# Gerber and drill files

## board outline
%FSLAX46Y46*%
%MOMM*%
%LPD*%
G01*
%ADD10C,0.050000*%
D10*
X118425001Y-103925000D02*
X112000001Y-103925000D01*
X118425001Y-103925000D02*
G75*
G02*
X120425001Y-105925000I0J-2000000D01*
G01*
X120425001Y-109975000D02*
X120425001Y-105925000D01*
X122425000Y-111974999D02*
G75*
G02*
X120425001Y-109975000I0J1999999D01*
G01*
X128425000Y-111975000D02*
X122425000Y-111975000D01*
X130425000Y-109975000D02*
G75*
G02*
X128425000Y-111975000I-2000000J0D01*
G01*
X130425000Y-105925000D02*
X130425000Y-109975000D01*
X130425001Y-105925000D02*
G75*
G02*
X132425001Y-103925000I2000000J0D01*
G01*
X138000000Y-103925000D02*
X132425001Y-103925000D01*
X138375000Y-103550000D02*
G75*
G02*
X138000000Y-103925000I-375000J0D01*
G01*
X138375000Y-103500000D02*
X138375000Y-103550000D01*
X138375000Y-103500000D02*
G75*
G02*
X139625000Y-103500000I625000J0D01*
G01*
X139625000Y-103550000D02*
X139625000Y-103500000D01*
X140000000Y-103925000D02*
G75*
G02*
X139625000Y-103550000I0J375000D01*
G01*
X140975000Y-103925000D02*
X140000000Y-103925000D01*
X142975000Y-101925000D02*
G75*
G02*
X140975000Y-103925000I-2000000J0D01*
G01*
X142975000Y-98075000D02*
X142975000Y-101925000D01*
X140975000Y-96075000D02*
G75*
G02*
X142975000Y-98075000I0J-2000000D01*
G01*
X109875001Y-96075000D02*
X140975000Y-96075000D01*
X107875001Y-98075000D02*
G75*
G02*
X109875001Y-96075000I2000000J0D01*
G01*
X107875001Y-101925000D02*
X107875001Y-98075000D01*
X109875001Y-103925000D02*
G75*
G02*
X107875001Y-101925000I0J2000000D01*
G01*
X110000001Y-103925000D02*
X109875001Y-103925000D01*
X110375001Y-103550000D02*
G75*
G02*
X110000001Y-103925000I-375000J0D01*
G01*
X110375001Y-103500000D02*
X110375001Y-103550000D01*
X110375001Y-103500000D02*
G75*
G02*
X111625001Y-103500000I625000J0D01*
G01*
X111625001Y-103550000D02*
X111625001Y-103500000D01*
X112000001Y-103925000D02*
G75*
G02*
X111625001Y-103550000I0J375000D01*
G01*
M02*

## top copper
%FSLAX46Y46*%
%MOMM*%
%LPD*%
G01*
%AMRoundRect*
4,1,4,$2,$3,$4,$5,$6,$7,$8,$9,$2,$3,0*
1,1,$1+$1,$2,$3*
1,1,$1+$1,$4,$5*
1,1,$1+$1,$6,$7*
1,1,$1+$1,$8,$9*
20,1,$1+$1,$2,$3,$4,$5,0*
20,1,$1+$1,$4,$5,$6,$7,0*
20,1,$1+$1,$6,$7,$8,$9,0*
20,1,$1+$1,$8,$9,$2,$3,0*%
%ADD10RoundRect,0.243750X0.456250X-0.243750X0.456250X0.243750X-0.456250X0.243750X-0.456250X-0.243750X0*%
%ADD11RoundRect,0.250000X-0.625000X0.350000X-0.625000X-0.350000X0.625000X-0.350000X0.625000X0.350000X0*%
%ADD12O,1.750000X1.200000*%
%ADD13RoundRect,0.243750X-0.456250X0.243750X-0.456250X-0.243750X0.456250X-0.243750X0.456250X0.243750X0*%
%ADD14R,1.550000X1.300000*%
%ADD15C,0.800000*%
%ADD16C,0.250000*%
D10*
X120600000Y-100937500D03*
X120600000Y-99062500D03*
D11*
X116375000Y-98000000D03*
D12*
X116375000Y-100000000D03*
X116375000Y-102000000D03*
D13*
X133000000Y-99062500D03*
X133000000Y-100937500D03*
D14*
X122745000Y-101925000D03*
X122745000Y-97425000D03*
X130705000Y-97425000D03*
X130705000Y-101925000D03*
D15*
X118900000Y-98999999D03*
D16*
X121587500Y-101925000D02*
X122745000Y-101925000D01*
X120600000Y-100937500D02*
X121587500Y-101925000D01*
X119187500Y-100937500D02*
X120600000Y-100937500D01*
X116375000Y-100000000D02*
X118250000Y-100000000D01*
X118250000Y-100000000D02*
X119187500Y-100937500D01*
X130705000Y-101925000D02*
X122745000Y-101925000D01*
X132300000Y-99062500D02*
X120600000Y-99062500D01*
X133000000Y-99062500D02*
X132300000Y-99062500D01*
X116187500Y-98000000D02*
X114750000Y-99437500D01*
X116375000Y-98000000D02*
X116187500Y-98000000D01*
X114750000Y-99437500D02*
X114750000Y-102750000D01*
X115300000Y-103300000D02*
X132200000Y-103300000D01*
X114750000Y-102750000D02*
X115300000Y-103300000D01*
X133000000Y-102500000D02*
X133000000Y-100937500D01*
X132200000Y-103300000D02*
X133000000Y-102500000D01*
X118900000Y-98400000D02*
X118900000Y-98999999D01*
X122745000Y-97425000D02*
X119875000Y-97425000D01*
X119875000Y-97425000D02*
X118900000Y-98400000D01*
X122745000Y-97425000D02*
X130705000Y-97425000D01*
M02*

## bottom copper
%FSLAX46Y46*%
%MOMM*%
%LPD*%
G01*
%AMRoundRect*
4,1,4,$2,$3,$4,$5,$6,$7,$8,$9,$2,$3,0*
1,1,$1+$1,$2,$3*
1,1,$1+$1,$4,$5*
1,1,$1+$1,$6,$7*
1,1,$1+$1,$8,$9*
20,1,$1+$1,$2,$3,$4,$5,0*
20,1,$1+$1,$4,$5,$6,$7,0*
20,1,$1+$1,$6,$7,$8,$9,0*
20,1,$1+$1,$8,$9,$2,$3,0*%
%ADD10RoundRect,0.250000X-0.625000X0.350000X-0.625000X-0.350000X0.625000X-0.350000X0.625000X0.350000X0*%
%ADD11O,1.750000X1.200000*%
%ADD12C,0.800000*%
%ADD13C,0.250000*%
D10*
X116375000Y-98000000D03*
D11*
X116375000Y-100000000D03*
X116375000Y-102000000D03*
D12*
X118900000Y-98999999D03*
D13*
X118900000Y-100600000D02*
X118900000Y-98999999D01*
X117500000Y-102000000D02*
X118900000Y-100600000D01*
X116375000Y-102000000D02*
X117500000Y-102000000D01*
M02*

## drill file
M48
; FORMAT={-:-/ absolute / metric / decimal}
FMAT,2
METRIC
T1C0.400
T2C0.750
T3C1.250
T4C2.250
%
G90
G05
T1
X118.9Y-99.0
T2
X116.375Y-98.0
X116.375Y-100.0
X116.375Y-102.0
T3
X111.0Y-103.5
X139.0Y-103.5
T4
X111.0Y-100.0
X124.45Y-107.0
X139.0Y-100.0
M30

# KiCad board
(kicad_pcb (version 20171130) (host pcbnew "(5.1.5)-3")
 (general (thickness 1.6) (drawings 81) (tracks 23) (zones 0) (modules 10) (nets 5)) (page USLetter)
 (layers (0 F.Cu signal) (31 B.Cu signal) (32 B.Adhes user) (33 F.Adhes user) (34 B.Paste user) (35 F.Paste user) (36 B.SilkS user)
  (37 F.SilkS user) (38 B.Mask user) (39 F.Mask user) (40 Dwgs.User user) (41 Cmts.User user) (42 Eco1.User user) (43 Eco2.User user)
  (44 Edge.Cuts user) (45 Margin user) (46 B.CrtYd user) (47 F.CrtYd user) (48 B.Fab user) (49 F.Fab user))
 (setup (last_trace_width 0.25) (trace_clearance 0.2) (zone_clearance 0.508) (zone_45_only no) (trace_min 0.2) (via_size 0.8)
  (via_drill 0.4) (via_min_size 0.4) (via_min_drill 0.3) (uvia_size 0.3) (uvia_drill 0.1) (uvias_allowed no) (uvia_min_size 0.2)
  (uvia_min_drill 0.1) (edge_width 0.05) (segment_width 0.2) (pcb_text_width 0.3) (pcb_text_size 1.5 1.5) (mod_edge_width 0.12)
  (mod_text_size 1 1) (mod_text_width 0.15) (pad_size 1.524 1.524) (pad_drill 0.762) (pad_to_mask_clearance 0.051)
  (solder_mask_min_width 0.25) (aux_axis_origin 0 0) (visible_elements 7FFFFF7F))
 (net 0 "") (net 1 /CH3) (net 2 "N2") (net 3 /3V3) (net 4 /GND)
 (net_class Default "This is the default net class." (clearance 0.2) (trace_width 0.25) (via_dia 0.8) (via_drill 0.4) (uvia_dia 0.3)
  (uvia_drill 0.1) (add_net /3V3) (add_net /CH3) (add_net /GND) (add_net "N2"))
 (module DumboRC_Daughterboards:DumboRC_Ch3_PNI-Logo (layer B.Cu) (at 128.5 100.25 180)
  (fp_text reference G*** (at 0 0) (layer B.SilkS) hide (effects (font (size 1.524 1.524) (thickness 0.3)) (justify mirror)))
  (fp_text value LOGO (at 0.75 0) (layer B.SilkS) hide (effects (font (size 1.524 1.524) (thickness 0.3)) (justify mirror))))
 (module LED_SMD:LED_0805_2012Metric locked (layer F.Cu) (at 120.6 100 90)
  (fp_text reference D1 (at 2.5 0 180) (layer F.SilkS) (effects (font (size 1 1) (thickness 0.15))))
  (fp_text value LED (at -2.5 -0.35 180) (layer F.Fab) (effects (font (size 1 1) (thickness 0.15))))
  (pad 1 smd roundrect (at -0.9375 0 90) (size 0.975 1.4) (layers F.Cu F.Paste F.Mask) (roundrect_rratio 0.25) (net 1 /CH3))
  (pad 2 smd roundrect (at 0.9375 0 90) (size 0.975 1.4) (layers F.Cu F.Paste F.Mask) (roundrect_rratio 0.25) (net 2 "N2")))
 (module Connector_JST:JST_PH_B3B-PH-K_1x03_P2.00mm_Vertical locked (layer F.Cu) (at 116.375 98 270)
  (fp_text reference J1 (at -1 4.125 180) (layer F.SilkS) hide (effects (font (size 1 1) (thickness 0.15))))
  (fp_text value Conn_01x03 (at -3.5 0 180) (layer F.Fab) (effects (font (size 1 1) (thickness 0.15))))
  (pad 1 thru_hole roundrect (at 0 0 270) (size 1.2 1.75) (drill 0.75) (layers *.Cu *.Mask) (roundrect_rratio 0.208333) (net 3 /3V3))
  (pad 2 thru_hole oval (at 2 0 270) (size 1.2 1.75) (drill 0.75) (layers *.Cu *.Mask) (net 1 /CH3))
  (pad 3 thru_hole oval (at 4 0 270) (size 1.2 1.75) (drill 0.75) (layers *.Cu *.Mask) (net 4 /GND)))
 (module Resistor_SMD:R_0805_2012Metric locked (layer F.Cu) (at 133 100 270)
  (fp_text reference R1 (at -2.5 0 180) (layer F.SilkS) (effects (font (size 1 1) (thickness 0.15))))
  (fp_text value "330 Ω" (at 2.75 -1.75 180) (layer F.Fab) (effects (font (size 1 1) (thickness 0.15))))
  (pad 1 smd roundrect (at -0.9375 0 270) (size 0.975 1.4) (layers F.Cu F.Paste F.Mask) (roundrect_rratio 0.25) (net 2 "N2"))
  (pad 2 smd roundrect (at 0.9375 0 270) (size 0.975 1.4) (layers F.Cu F.Paste F.Mask) (roundrect_rratio 0.25) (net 3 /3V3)))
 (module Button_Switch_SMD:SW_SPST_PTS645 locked (layer F.Cu) (at 126.725 99.675)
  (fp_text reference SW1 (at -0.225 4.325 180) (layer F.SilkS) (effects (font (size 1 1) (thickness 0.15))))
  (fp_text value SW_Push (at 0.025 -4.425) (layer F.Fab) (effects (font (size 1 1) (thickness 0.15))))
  (pad 2 smd rect (at -3.98 2.25) (size 1.55 1.3) (layers F.Cu F.Paste F.Mask) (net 1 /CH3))
  (pad 1 smd rect (at -3.98 -2.25) (size 1.55 1.3) (layers F.Cu F.Paste F.Mask) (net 4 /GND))
  (pad 1 smd rect (at 3.98 -2.25) (size 1.55 1.3) (layers F.Cu F.Paste F.Mask) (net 4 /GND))
  (pad 2 smd rect (at 3.98 2.25) (size 1.55 1.3) (layers F.Cu F.Paste F.Mask) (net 1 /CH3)))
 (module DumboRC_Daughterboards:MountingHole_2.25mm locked (layer F.Cu) (at 111 100)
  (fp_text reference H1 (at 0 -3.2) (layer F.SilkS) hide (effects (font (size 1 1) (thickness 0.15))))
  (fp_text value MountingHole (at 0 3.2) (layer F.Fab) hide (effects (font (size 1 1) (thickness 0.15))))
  (pad "" np_thru_hole circle (at 0 0 90) (size 2.25 2.25) (drill 2.25) (layers *.Cu *.Mask)))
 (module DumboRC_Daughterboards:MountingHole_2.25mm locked (layer F.Cu) (at 139 100)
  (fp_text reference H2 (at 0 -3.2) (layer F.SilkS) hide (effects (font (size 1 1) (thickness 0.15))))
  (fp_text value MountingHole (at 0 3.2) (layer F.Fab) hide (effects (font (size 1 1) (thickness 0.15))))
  (pad "" np_thru_hole circle (at 0 0 90) (size 2.25 2.25) (drill 2.25) (layers *.Cu *.Mask)))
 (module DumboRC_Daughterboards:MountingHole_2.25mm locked (layer F.Cu) (at 124.45 107)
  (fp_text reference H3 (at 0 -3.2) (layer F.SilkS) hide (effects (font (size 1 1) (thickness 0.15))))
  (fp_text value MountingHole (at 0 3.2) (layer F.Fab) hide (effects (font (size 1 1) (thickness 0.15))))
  (pad "" np_thru_hole circle (at 0 0 90) (size 2.25 2.25) (drill 2.25) (layers *.Cu *.Mask)))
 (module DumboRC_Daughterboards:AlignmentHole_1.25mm (layer F.Cu) (at 111 103.5)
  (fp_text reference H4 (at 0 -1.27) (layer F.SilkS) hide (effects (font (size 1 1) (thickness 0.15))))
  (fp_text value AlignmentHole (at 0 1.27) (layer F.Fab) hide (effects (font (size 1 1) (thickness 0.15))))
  (pad "" np_thru_hole circle (at 0 0 90) (size 1.25 1.25) (drill 1.25) (layers *.Cu *.Mask)))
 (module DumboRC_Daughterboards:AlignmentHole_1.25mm (layer F.Cu) (at 139 103.5)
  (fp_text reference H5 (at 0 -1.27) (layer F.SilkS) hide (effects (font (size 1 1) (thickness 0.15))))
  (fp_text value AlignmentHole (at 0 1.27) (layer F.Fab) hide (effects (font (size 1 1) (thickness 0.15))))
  (pad "" np_thru_hole circle (at 0 0 90) (size 1.25 1.25) (drill 1.25) (layers *.Cu *.Mask)))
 (gr_line (start 118.425001 103.925) (end 112.000001 103.925) (layer Edge.Cuts) (width 0.05))
 (gr_arc (start 118.425001 105.925) (end 120.425001 105.925) (angle -90) (layer Edge.Cuts) (width 0.05))
 (gr_line (start 120.425001 109.975) (end 120.425001 105.925) (layer Edge.Cuts) (width 0.05))
 (gr_arc (start 122.425 109.975) (end 120.425001 109.975) (angle -90) (layer Edge.Cuts) (width 0.05))
 (gr_line (start 128.425 111.975) (end 122.425 111.975) (layer Edge.Cuts) (width 0.05))
 (gr_arc (start 128.425 109.975) (end 128.425 111.975) (angle -90) (layer Edge.Cuts) (width 0.05))
 (gr_line (start 130.425 105.925) (end 130.425 109.975) (layer Edge.Cuts) (width 0.05))
 (gr_arc (start 132.425001 105.925) (end 132.425001 103.925) (angle -90) (layer Edge.Cuts) (width 0.05))
 (gr_line (start 138 103.925) (end 132.425001 103.925) (layer Edge.Cuts) (width 0.05))
 (gr_arc (start 138 103.55) (end 138 103.925) (angle -90) (layer Edge.Cuts) (width 0.05))
 (gr_line (start 138.375 103.5) (end 138.375 103.55) (layer Edge.Cuts) (width 0.05))
 (gr_arc (start 139 103.5) (end 139.625 103.5) (angle -180) (layer Edge.Cuts) (width 0.05))
 (gr_line (start 139.625 103.55) (end 139.625 103.5) (layer Edge.Cuts) (width 0.05))
 (gr_arc (start 140 103.55) (end 139.625 103.55) (angle -90) (layer Edge.Cuts) (width 0.05))
 (gr_line (start 140.975 103.925) (end 140 103.925) (layer Edge.Cuts) (width 0.05))
 (gr_arc (start 140.975 101.925) (end 140.975 103.925) (angle -90) (layer Edge.Cuts) (width 0.05))
 (gr_line (start 142.975 98.075) (end 142.975 101.925) (layer Edge.Cuts) (width 0.05))
 (gr_arc (start 140.975 98.075) (end 142.975 98.075) (angle -90) (layer Edge.Cuts) (width 0.05))
 (gr_line (start 109.875001 96.075) (end 140.975 96.075) (layer Edge.Cuts) (width 0.05))
 (gr_arc (start 109.875001 98.075) (end 109.875001 96.075) (angle -90) (layer Edge.Cuts) (width 0.05))
 (gr_line (start 107.875001 101.925) (end 107.875001 98.075) (layer Edge.Cuts) (width 0.05))
 (gr_arc (start 109.875001 101.925) (end 107.875001 101.925) (angle -90) (layer Edge.Cuts) (width 0.05))
 (gr_line (start 110.000001 103.925) (end 109.875001 103.925) (layer Edge.Cuts) (width 0.05))
 (gr_arc (start 110.000001 103.55) (end 110.000001 103.925) (angle -90) (layer Edge.Cuts) (width 0.05))
 (gr_line (start 110.375001 103.5) (end 110.375001 103.55) (layer Edge.Cuts) (width 0.05))
 (gr_arc (start 111.000001 103.5) (end 111.625001 103.5) (angle -180) (layer Edge.Cuts) (width 0.05))
 (gr_line (start 111.625001 103.55) (end 111.625001 103.5) (layer Edge.Cuts) (width 0.05))
 (gr_arc (start 112.000001 103.55) (end 111.625001 103.55) (angle -90) (layer Edge.Cuts) (width 0.05))
 (segment (start 121.5875 101.925) (end 122.745 101.925) (width 0.25) (layer F.Cu) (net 1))
 (segment (start 120.6 100.9375) (end 121.5875 101.925) (width 0.25) (layer F.Cu) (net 1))
 (segment (start 119.1875 100.9375) (end 120.6 100.9375) (width 0.25) (layer F.Cu) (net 1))
 (segment (start 116.375 100) (end 118.25 100) (width 0.25) (layer F.Cu) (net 1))
 (segment (start 118.25 100) (end 119.1875 100.9375) (width 0.25) (layer F.Cu) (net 1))
 (segment (start 130.705 101.925) (end 122.745 101.925) (width 0.25) (layer F.Cu) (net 1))
 (segment (start 132.3 99.0625) (end 120.6 99.0625) (width 0.25) (layer F.Cu) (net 2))
 (segment (start 133 99.0625) (end 132.3 99.0625) (width 0.25) (layer F.Cu) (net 2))
 (segment (start 116.1875 98) (end 114.75 99.4375) (width 0.25) (layer F.Cu) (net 3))
 (segment (start 116.375 98) (end 116.1875 98) (width 0.25) (layer F.Cu) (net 3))
 (segment (start 114.75 99.4375) (end 114.75 102.75) (width 0.25) (layer F.Cu) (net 3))
 (segment (start 115.3 103.3) (end 132.2 103.3) (width 0.25) (layer F.Cu) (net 3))
 (segment (start 114.75 102.75) (end 115.3 103.3) (width 0.25) (layer F.Cu) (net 3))
 (segment (start 133 102.5) (end 133 100.9375) (width 0.25) (layer F.Cu) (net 3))
 (segment (start 132.2 103.3) (end 133 102.5) (width 0.25) (layer F.Cu) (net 3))
 (via (at 118.9 98.999999) (size 0.8) (drill 0.4) (layers F.Cu B.Cu) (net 4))
 (segment (start 118.9 100.6) (end 118.9 98.999999) (width 0.25) (layer B.Cu) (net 4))
 (segment (start 117.5 102) (end 118.9 100.6) (width 0.25) (layer B.Cu) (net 4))
 (segment (start 116.375 102) (end 117.5 102) (width 0.25) (layer B.Cu) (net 4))
 (segment (start 118.9 98.4) (end 118.9 98.999999) (width 0.25) (layer F.Cu) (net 4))
 (segment (start 122.745 97.425) (end 119.875 97.425) (width 0.25) (layer F.Cu) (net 4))
 (segment (start 119.875 97.425) (end 118.9 98.4) (width 0.25) (layer F.Cu) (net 4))
 (segment (start 122.745 97.425) (end 130.705 97.425) (width 0.25) (layer F.Cu) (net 4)))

